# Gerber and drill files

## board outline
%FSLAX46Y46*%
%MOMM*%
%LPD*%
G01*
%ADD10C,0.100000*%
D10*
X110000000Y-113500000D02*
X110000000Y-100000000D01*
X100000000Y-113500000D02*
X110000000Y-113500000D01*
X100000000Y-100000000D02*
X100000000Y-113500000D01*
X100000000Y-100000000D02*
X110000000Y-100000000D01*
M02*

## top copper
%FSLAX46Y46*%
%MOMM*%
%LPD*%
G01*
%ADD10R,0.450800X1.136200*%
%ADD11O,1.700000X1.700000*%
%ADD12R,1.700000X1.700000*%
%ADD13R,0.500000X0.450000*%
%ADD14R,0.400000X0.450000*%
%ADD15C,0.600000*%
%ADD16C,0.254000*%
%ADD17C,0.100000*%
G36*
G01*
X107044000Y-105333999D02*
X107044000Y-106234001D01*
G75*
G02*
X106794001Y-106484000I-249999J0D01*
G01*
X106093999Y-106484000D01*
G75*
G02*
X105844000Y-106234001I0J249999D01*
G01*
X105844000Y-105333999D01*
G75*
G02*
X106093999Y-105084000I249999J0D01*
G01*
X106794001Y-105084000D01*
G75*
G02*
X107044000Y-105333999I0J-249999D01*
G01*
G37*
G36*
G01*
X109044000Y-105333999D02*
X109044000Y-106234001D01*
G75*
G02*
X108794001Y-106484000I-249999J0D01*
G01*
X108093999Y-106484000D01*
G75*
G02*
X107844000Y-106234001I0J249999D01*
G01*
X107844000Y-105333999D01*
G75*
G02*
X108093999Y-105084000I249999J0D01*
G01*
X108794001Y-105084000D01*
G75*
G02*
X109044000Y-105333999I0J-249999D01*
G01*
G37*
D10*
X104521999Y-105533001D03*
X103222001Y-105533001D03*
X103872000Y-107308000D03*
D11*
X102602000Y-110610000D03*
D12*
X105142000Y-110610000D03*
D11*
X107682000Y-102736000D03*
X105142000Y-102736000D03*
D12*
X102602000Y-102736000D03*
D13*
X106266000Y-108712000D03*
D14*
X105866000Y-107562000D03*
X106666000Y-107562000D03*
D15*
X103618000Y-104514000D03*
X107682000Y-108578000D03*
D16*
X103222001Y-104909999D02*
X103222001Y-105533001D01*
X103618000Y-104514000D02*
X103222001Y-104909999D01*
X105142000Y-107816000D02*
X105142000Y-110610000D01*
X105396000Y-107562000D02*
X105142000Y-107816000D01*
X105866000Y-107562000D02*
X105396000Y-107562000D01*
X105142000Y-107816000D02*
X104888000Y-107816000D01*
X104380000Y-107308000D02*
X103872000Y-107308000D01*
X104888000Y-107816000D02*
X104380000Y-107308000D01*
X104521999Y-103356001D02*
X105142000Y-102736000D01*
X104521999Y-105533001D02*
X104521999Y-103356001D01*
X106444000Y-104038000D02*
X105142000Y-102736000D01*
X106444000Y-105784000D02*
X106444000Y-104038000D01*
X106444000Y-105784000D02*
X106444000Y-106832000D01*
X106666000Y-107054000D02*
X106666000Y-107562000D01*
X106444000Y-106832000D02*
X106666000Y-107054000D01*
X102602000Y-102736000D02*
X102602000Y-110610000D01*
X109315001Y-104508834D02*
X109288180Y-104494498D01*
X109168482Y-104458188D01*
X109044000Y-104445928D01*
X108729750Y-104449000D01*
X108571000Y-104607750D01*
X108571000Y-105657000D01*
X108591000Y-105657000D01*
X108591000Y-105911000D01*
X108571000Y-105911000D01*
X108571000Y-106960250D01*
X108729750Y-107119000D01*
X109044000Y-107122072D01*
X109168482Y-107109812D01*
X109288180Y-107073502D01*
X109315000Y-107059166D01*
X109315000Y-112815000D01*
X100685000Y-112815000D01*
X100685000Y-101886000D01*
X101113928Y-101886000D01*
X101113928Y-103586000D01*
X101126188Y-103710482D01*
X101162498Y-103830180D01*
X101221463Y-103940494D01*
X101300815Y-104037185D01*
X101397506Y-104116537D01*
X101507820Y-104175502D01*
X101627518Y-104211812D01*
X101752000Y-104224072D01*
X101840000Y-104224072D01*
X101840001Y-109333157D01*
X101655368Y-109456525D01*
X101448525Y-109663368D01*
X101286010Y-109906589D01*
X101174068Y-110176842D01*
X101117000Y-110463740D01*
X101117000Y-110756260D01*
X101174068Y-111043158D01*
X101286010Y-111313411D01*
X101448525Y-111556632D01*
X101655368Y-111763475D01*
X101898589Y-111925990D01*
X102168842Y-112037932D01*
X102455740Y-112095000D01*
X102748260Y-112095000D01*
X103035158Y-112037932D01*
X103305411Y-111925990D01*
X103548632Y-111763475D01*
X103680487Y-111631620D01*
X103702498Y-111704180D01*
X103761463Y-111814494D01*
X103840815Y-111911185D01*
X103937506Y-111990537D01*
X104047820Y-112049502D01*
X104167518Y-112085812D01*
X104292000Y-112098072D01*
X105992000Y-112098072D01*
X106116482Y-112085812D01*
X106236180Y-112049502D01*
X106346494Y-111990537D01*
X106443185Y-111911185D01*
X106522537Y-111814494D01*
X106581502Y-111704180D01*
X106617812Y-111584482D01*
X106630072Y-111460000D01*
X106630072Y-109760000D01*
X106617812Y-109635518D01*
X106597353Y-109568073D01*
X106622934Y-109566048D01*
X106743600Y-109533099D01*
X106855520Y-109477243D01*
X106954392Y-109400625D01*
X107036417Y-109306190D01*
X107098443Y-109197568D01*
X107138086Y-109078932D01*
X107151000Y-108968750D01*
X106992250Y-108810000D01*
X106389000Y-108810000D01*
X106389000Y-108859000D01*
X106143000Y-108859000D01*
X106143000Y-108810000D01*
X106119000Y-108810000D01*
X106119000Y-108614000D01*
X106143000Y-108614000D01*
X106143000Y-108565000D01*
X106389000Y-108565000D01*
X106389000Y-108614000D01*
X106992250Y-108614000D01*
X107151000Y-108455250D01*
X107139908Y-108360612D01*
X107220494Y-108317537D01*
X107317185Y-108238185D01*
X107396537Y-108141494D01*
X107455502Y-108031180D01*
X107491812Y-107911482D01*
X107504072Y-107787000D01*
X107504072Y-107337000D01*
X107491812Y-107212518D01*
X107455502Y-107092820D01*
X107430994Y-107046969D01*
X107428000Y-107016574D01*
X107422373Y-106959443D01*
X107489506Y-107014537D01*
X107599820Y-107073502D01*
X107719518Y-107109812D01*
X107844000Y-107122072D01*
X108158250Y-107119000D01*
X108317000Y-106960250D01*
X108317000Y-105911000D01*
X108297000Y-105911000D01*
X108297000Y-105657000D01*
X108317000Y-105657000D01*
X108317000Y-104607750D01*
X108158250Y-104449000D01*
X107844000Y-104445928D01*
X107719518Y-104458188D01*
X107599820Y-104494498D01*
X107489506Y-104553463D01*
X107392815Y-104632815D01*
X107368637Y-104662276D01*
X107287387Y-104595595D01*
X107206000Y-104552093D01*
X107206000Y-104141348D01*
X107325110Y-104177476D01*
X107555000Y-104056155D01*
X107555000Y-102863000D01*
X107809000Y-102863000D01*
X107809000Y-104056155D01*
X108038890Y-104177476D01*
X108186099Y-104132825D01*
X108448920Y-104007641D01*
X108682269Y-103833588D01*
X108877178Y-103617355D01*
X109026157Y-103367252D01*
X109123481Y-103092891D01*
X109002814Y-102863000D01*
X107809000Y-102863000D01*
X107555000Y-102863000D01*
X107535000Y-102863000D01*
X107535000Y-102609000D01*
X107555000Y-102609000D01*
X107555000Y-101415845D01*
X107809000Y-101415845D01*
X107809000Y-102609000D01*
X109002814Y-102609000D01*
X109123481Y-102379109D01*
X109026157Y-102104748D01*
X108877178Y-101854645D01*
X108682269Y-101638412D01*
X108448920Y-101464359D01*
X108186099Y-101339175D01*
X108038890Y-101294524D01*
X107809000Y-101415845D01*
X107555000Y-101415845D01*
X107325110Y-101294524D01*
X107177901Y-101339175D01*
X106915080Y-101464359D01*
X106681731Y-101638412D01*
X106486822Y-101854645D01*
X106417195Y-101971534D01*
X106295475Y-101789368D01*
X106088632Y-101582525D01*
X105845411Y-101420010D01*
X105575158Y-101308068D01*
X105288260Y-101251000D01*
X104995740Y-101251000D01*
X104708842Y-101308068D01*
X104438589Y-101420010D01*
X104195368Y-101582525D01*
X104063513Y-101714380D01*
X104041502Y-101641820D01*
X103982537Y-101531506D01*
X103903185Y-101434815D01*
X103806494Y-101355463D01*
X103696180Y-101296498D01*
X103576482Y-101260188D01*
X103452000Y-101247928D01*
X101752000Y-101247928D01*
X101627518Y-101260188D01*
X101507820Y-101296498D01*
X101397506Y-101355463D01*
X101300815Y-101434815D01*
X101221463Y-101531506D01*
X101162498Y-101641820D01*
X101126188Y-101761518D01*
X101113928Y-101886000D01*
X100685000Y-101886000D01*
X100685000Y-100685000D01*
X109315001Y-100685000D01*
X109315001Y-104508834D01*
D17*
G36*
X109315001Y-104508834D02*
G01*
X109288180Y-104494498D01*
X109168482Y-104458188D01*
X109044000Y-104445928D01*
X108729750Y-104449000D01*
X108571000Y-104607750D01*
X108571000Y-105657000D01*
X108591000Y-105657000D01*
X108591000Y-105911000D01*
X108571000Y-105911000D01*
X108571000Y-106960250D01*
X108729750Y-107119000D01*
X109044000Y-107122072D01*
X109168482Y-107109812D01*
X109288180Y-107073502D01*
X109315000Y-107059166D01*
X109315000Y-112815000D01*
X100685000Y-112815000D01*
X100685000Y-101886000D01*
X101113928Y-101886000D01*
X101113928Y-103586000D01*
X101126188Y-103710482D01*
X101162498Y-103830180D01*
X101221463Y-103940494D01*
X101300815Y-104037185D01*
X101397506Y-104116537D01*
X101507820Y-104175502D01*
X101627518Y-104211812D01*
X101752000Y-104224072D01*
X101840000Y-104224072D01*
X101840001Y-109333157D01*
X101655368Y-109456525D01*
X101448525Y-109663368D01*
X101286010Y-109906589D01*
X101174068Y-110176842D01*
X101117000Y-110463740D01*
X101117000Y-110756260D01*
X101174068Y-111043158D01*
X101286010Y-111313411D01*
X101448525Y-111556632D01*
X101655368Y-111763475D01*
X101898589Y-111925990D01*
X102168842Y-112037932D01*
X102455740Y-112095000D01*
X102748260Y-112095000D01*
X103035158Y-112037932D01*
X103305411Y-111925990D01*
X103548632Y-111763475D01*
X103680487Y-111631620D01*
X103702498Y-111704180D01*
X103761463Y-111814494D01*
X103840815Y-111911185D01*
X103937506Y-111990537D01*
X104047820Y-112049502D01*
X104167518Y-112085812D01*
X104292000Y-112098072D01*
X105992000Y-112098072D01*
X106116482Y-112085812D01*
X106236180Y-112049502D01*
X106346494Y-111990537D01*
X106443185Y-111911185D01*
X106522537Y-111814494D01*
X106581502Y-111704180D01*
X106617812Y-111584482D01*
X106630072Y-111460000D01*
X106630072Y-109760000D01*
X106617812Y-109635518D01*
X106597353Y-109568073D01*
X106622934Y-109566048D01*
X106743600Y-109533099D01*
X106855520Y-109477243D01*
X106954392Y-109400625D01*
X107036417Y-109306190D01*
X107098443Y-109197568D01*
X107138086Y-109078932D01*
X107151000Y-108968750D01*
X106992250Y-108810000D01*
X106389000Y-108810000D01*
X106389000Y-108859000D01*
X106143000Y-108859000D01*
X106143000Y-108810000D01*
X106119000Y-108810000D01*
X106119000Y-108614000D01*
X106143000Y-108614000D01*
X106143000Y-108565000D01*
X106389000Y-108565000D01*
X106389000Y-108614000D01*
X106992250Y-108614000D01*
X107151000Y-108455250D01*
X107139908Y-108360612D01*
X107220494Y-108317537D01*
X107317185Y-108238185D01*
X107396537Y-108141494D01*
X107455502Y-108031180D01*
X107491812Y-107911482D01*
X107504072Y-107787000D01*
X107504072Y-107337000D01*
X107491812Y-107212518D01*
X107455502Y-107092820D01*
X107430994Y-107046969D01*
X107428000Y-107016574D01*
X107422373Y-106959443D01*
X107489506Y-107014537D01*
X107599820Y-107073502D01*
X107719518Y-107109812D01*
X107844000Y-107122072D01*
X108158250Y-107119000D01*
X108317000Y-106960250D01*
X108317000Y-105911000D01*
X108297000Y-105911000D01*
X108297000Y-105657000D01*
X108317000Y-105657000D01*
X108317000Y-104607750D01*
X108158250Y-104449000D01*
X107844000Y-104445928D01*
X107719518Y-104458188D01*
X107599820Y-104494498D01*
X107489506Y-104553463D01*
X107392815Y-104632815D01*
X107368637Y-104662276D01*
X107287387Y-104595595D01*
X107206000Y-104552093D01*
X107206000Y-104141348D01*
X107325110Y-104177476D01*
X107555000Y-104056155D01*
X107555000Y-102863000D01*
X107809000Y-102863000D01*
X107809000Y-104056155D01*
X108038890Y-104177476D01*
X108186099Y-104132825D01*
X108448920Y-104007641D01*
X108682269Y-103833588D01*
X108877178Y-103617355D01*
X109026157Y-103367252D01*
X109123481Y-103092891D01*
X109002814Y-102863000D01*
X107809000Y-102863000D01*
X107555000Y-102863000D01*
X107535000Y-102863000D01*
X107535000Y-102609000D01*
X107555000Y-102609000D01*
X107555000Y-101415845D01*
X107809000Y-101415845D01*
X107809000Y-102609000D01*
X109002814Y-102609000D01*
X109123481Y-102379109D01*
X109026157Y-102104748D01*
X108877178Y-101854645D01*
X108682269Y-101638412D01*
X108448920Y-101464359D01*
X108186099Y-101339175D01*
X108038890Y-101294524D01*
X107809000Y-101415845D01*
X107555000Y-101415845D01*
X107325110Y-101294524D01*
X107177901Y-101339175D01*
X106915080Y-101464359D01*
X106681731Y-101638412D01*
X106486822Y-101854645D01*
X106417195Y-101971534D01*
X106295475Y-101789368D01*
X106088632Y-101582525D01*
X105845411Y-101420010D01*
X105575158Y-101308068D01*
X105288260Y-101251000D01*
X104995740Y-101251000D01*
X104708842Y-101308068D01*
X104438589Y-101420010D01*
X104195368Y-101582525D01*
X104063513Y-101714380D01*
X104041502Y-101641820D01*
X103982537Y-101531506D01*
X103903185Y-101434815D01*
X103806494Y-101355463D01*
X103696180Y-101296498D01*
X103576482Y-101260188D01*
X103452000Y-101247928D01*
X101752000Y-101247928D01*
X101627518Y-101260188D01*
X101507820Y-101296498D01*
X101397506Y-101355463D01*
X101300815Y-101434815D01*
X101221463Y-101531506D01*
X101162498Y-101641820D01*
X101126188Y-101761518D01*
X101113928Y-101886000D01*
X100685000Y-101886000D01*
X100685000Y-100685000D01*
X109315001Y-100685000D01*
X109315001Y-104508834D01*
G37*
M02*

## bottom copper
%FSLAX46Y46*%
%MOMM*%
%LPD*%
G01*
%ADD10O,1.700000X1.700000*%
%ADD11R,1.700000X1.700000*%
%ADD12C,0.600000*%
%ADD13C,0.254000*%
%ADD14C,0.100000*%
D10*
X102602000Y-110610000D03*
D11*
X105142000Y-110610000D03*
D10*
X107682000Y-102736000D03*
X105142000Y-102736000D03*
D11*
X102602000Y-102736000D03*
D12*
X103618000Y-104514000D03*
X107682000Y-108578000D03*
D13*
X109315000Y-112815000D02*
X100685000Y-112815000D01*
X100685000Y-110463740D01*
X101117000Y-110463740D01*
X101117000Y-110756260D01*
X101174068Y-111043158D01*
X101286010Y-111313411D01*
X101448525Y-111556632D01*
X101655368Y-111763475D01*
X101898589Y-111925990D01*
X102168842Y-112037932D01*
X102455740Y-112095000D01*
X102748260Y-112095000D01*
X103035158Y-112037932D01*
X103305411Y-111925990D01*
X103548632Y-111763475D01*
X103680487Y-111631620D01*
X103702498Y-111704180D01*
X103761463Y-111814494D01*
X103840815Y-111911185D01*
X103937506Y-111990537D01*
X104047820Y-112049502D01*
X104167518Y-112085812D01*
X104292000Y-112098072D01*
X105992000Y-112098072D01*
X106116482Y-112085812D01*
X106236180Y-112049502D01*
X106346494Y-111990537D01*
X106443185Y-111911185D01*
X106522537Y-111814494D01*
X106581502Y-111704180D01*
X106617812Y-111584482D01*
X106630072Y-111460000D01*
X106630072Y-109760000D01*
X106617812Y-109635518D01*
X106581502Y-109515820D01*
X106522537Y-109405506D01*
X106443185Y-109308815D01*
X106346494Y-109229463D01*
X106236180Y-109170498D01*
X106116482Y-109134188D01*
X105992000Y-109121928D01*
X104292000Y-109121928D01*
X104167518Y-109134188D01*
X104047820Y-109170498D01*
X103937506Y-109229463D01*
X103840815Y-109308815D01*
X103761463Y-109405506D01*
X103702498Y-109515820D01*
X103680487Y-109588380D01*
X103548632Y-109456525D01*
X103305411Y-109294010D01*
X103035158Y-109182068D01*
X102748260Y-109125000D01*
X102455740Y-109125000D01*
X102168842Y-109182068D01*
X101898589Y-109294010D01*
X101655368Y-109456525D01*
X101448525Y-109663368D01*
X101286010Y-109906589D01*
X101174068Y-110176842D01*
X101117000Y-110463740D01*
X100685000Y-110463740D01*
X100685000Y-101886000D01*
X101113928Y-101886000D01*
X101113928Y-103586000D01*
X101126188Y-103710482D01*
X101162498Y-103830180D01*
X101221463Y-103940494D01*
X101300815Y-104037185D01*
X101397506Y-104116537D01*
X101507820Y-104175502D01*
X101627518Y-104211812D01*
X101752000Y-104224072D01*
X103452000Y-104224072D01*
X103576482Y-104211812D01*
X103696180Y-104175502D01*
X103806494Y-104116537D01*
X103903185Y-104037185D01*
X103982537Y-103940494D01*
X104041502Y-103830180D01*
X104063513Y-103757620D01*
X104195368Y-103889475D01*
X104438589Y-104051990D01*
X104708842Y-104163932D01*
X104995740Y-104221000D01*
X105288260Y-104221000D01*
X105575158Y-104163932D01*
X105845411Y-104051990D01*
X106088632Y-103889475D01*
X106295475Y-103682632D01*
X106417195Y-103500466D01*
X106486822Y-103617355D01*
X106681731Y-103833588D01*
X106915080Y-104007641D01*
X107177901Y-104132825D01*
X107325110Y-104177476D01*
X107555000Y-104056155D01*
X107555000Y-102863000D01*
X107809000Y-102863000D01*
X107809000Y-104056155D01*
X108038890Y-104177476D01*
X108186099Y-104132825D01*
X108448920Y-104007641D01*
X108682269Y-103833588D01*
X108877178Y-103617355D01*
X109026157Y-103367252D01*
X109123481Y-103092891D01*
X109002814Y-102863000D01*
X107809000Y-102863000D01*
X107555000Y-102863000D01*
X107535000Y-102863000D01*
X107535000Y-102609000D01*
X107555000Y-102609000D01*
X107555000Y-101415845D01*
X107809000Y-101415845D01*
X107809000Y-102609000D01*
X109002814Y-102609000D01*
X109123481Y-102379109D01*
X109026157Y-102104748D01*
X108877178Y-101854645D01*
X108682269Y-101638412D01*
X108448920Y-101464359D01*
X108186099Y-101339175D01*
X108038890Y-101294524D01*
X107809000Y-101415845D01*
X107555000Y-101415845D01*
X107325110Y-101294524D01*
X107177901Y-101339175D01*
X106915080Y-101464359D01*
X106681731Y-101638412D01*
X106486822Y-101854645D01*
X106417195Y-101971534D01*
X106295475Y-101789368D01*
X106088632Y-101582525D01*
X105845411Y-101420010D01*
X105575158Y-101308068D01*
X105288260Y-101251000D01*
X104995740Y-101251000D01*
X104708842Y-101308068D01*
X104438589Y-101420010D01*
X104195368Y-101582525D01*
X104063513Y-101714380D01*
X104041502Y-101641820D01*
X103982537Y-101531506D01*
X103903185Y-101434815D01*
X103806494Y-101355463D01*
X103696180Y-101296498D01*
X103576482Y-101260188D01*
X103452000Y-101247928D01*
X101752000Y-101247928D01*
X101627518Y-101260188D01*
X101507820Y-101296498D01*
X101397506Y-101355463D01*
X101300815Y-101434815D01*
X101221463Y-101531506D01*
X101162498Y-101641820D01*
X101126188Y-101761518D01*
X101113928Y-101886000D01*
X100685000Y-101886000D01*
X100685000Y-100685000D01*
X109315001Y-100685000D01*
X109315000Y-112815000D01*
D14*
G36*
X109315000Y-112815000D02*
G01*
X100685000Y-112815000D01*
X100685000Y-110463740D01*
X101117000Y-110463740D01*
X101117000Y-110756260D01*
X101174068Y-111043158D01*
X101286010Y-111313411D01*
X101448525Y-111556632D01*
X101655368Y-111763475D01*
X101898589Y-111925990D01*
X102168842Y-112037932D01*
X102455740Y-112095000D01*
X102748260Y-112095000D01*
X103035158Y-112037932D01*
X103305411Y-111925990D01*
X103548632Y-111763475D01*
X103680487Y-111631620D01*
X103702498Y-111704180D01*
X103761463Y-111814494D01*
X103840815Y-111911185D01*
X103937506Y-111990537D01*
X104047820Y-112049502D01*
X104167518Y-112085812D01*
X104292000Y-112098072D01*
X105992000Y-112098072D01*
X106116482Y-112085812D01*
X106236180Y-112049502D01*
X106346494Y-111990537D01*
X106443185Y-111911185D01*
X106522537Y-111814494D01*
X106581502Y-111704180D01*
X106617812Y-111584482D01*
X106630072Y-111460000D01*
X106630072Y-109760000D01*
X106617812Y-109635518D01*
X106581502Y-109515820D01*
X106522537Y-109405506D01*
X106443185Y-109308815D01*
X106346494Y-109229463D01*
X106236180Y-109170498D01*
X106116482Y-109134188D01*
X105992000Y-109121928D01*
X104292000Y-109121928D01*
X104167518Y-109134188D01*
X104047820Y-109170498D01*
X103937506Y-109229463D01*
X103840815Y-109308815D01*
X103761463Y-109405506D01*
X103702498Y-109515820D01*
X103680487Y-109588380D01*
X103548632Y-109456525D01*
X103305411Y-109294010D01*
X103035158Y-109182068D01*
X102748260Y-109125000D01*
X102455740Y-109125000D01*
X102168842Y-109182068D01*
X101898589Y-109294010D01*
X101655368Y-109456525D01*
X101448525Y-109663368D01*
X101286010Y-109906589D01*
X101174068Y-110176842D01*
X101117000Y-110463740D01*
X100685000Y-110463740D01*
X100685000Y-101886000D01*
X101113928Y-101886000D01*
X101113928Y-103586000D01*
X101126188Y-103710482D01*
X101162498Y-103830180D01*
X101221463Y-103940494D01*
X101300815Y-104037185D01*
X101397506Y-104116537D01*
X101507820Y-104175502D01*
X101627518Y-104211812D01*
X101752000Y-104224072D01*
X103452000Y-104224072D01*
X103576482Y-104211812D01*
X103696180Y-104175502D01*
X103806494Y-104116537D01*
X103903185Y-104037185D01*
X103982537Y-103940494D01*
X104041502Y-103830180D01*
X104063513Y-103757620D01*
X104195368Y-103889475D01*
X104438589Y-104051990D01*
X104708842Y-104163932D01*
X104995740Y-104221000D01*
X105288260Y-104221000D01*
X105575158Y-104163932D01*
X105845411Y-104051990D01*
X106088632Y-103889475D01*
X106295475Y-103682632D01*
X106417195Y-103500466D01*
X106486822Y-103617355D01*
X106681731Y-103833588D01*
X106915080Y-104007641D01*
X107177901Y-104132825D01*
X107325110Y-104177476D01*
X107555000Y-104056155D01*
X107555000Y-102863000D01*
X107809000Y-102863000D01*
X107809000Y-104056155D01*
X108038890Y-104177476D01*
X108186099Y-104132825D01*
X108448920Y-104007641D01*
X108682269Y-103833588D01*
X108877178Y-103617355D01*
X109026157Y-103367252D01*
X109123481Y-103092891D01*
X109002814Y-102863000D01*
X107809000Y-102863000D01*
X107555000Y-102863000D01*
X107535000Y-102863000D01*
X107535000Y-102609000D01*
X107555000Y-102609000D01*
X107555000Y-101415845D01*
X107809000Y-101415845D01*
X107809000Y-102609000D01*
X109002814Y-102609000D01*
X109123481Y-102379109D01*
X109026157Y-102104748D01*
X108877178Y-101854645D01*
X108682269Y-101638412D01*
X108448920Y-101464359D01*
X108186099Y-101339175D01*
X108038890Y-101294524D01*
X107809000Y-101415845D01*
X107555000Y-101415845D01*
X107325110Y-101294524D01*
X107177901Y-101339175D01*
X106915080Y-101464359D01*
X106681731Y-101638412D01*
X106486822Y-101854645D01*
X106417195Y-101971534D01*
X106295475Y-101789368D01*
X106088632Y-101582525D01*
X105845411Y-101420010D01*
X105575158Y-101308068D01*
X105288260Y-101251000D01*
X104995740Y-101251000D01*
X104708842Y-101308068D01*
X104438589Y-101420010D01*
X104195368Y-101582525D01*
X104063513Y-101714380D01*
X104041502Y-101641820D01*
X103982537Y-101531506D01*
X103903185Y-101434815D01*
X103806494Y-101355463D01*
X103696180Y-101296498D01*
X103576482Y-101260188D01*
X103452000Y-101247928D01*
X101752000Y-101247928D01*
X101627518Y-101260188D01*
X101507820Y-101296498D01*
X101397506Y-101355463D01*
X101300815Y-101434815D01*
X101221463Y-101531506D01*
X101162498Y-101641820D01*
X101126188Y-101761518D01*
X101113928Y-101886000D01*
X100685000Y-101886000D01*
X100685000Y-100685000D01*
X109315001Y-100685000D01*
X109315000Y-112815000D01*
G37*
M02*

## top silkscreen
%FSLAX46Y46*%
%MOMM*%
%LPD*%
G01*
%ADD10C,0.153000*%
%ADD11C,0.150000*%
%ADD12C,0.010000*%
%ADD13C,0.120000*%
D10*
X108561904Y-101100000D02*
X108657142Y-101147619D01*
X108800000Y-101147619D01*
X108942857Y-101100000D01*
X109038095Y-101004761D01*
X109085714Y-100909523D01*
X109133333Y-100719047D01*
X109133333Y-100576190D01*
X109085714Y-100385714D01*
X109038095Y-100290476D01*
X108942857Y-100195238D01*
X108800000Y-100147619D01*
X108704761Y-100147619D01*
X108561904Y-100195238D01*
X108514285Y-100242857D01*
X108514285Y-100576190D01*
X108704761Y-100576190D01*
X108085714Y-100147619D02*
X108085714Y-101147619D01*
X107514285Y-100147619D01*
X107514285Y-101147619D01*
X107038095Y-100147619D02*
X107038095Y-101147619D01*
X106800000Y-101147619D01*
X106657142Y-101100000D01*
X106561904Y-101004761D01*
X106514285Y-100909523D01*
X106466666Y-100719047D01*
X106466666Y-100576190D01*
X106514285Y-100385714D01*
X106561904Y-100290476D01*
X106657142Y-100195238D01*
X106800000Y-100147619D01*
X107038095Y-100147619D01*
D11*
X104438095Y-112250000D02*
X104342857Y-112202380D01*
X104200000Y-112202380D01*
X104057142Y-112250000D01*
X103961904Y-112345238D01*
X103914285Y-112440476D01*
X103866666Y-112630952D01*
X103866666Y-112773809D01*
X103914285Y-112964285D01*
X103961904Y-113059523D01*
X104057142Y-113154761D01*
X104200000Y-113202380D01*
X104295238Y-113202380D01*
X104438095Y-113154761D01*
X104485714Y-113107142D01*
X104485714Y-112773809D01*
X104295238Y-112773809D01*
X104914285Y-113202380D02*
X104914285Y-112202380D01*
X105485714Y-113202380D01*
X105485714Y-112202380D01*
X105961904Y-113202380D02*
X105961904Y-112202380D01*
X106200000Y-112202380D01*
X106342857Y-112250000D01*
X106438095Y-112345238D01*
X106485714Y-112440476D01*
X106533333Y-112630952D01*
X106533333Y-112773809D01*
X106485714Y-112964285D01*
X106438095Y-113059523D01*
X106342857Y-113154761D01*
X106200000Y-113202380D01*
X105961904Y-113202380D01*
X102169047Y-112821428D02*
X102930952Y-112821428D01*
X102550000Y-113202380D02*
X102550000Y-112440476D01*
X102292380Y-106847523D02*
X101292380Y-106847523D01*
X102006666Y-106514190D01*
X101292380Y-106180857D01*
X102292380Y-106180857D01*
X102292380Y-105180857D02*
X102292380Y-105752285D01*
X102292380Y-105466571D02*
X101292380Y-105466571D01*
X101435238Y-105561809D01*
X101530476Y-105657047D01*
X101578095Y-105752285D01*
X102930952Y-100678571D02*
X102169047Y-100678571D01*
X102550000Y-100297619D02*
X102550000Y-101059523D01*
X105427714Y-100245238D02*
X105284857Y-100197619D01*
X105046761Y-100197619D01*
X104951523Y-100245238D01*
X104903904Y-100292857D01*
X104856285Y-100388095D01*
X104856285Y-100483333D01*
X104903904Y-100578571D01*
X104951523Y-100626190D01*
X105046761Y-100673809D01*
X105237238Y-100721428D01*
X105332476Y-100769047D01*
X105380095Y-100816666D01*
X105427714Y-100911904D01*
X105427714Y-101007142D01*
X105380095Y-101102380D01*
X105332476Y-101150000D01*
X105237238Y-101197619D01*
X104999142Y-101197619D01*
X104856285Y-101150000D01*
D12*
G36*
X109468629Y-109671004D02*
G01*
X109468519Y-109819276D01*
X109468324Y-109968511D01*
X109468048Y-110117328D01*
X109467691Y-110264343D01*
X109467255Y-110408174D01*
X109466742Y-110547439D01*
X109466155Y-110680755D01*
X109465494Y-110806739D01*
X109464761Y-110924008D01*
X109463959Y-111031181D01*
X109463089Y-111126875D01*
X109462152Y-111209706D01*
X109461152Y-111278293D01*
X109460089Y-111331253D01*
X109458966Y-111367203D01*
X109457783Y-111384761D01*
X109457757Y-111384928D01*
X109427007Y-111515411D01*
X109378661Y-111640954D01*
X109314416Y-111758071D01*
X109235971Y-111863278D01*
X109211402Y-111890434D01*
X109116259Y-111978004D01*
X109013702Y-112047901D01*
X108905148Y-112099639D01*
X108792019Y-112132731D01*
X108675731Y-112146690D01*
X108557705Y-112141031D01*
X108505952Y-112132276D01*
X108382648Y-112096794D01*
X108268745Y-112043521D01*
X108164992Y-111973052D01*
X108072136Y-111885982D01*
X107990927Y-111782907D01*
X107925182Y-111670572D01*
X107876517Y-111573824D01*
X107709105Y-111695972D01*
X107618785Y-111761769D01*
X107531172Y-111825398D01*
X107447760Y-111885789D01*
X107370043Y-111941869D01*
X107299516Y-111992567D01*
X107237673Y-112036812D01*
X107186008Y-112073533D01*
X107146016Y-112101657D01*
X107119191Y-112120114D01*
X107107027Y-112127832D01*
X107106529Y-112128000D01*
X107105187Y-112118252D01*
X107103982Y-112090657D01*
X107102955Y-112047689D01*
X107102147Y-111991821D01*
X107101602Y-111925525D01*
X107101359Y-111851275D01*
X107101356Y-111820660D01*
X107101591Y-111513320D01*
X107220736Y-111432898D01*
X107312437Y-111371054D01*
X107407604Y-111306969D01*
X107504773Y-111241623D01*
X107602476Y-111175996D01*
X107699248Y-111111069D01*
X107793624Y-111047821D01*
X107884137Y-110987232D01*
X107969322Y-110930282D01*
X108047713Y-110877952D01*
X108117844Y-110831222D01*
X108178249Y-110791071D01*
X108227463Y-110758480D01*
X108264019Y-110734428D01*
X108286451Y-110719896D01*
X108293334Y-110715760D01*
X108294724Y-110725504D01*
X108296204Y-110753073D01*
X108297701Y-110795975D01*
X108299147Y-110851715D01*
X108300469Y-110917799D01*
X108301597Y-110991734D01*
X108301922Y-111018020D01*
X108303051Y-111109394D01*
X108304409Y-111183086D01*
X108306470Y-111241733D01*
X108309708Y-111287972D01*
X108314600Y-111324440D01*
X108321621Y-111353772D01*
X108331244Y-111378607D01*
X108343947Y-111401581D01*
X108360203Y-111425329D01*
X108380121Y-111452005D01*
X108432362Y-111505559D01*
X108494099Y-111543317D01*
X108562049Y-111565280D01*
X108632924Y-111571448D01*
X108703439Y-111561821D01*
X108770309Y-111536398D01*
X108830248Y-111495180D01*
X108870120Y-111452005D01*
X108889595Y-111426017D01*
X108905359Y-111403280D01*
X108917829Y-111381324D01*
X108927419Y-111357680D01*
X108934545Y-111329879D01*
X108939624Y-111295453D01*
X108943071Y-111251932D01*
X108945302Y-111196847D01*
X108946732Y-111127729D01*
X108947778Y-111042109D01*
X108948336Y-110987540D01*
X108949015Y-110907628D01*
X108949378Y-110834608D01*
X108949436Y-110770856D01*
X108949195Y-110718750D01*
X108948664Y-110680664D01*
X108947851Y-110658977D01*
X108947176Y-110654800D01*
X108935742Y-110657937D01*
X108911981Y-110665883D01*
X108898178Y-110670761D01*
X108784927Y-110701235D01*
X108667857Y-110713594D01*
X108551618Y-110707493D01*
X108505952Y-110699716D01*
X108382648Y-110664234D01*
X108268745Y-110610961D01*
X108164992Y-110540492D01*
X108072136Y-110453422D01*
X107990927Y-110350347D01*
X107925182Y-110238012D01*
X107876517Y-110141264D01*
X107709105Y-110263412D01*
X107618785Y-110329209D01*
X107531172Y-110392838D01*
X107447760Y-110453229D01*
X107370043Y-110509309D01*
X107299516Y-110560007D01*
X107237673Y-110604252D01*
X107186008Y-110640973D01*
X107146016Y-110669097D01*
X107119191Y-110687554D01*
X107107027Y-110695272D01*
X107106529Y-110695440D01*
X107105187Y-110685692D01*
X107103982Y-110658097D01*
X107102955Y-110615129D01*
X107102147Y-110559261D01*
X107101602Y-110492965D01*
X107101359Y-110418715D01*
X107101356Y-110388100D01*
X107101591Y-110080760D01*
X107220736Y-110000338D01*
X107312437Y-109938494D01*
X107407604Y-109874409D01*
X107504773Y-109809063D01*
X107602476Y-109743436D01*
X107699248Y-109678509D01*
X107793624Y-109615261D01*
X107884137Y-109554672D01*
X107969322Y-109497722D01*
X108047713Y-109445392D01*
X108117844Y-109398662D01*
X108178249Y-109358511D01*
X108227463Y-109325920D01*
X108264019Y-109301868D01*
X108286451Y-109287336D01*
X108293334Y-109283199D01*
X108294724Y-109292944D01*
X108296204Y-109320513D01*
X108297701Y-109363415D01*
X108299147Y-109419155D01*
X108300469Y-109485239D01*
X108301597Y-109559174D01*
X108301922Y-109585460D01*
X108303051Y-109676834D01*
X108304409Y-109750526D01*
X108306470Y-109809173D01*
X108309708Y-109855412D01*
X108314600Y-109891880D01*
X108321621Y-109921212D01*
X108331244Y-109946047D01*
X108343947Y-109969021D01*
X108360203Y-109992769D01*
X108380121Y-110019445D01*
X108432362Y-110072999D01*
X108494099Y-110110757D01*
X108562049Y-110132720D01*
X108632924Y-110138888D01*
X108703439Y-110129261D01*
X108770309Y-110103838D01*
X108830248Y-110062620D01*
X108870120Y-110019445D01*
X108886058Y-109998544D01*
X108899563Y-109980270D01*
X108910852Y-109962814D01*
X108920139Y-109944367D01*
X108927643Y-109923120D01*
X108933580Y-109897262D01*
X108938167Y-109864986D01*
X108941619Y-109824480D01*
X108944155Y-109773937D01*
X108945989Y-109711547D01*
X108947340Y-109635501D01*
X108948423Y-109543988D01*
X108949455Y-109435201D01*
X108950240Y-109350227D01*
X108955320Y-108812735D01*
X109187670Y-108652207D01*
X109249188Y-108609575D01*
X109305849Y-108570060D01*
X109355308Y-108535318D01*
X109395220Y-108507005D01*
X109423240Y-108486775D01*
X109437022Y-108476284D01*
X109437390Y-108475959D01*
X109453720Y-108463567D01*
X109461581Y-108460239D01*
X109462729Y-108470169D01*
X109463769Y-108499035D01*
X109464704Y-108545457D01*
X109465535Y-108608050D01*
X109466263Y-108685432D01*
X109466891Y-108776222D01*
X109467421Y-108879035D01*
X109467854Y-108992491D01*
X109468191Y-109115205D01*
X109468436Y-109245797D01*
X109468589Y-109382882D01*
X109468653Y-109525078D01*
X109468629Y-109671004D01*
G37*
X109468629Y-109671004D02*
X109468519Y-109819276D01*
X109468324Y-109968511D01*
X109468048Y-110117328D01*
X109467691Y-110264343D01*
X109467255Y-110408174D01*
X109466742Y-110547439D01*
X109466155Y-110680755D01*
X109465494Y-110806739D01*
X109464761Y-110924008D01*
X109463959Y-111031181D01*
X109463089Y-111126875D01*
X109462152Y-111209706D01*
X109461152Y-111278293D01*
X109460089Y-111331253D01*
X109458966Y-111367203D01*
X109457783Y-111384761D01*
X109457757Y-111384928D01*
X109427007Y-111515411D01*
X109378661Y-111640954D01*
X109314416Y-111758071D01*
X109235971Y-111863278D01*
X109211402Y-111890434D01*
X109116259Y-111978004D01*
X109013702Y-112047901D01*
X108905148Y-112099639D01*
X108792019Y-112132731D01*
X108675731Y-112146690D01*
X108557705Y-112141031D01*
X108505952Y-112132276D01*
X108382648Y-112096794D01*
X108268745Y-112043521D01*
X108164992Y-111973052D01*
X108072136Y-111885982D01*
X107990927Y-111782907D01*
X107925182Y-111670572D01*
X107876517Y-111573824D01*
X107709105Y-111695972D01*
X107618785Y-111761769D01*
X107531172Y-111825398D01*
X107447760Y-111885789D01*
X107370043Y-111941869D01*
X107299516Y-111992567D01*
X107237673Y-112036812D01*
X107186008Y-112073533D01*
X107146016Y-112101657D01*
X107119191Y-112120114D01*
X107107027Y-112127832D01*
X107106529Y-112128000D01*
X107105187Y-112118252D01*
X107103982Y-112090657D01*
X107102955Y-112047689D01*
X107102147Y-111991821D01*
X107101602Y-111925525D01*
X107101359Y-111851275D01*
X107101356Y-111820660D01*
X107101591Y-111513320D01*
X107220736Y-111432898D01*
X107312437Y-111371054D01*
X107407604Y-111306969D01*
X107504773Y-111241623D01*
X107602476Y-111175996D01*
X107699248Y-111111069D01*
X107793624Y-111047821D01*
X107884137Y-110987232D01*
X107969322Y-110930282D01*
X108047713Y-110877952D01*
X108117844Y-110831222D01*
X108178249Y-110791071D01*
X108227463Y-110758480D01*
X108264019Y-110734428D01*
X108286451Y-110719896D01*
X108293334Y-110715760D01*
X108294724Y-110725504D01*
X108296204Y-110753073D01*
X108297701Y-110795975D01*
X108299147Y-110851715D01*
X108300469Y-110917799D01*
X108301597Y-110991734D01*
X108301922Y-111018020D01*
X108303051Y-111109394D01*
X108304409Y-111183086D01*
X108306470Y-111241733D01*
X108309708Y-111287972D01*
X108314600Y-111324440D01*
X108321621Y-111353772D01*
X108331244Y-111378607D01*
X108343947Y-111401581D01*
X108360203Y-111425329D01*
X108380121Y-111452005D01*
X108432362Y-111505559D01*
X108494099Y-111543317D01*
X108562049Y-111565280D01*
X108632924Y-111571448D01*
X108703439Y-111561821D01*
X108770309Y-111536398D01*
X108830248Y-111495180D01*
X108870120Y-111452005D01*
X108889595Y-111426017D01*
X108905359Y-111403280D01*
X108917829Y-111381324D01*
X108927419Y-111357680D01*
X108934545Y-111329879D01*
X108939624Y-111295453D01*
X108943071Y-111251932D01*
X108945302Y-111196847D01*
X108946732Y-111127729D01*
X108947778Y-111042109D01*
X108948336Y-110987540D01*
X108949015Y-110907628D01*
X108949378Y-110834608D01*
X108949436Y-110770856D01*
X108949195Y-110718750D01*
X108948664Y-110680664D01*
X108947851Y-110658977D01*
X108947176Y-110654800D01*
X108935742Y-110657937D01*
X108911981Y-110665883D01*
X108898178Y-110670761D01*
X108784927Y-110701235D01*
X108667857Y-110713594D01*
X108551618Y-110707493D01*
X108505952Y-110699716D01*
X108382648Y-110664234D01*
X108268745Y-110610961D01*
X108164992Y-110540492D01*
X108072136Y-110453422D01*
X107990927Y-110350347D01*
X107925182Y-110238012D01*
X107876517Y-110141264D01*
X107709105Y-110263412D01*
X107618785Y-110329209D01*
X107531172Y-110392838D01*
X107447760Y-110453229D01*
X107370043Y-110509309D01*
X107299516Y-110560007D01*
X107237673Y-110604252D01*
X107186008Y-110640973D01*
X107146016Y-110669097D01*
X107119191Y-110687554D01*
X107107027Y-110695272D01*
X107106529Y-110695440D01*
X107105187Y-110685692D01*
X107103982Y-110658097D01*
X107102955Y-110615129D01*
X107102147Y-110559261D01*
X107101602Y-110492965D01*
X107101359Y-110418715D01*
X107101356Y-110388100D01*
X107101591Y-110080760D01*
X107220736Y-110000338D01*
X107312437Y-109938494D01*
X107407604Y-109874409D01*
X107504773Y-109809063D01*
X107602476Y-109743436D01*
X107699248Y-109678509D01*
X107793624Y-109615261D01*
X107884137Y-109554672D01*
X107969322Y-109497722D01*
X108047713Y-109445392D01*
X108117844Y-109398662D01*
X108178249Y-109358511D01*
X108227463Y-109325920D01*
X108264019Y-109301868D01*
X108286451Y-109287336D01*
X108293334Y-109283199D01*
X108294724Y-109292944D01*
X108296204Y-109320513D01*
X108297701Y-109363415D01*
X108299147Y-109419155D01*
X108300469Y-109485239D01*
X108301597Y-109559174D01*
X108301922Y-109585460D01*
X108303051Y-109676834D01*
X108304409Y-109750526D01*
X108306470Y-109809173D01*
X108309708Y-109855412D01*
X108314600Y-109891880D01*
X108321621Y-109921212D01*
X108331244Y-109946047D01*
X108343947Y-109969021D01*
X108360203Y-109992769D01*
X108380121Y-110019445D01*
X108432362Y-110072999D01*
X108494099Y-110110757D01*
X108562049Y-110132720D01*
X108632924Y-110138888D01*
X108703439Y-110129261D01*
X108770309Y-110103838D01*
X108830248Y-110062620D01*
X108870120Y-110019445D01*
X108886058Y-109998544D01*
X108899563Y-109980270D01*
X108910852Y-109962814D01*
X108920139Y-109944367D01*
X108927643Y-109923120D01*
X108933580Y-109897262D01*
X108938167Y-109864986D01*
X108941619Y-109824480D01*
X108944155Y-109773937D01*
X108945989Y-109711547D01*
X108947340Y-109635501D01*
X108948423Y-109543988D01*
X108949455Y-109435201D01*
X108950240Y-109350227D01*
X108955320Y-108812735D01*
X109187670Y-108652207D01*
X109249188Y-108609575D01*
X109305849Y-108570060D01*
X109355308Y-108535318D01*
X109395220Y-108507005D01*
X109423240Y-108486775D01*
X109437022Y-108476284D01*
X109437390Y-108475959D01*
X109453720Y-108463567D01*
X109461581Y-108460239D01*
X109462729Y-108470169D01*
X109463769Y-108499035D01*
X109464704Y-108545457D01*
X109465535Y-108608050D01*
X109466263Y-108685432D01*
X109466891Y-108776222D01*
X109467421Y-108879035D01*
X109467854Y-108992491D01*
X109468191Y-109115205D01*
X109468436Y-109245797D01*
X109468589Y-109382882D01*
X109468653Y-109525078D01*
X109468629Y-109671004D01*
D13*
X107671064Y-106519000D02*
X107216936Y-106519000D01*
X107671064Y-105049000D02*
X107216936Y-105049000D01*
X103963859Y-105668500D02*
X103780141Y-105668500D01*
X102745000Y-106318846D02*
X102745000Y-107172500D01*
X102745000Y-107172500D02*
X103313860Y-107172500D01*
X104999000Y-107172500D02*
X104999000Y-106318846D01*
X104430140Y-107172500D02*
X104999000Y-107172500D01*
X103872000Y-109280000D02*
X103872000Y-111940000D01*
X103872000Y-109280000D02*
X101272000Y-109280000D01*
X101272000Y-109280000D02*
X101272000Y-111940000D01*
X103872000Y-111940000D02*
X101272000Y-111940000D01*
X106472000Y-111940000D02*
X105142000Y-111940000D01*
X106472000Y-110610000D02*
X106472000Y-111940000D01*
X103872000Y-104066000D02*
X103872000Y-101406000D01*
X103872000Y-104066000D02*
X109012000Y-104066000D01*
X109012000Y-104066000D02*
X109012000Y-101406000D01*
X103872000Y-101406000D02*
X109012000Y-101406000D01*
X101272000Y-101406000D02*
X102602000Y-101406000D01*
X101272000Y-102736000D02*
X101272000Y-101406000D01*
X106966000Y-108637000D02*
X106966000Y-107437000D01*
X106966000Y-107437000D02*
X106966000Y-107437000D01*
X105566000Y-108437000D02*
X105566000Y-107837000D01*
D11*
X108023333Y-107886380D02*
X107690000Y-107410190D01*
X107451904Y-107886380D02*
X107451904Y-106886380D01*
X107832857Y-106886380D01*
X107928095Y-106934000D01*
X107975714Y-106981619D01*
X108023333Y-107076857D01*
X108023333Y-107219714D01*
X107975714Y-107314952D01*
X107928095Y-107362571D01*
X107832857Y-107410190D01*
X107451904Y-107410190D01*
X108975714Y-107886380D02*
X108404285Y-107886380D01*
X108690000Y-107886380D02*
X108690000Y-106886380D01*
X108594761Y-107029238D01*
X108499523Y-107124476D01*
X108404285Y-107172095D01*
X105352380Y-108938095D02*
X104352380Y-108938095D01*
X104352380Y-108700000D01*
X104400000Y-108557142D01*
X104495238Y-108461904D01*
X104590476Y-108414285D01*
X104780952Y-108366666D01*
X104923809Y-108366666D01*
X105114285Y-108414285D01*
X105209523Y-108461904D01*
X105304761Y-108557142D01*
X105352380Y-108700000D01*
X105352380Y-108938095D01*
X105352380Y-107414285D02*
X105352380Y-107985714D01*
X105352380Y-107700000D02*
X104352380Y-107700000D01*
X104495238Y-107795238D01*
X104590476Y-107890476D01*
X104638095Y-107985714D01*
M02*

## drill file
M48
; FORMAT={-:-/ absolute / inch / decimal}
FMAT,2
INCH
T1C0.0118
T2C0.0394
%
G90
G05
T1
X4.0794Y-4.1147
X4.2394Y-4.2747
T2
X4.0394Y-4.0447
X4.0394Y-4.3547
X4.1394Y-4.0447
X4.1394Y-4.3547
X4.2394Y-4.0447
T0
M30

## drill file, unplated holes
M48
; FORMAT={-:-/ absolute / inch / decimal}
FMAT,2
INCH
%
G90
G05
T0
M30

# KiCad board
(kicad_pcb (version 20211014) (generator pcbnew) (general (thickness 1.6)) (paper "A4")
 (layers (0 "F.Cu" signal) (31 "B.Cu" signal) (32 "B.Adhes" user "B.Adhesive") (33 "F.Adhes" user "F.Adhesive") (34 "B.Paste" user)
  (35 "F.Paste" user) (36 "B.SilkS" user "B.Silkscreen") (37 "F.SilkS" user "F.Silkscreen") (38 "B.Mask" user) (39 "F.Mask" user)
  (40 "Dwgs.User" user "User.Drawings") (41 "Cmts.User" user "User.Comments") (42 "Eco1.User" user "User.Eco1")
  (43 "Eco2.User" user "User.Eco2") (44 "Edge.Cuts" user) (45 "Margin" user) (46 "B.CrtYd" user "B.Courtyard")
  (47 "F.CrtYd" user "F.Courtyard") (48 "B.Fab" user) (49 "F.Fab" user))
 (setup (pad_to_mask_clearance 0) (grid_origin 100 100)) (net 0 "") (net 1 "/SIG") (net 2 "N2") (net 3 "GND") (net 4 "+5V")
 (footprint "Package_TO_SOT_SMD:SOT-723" (layer "F.Cu") (at 106.266 108.137 -90)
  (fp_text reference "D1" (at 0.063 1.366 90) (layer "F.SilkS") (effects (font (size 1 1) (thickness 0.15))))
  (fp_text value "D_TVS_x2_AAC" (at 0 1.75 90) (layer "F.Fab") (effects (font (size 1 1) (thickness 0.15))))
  (fp_line (start 0.5 -0.7) (end -0.7 -0.7) (layer "F.SilkS") (width 0.12))
  (fp_line (start -0.7 -0.7) (end -0.7 -0.7) (layer "F.SilkS") (width 0.12))
  (fp_line (start 0.3 0.7) (end -0.3 0.7) (layer "F.SilkS") (width 0.12))
  (pad "1" smd rect locked (at -0.575 -0.4 270) (size 0.45 0.4) (layers "F.Cu" "F.Paste" "F.Mask") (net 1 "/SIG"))
  (pad "2" smd rect locked (at -0.575 0.4 270) (size 0.45 0.4) (layers "F.Cu" "F.Paste" "F.Mask") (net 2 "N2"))
  (pad "3" smd rect locked (at 0.575 0 270) (size 0.45 0.5) (layers "F.Cu" "F.Paste" "F.Mask") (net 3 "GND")))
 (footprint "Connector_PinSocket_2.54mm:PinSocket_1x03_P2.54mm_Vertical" (layer "F.Cu") (at 102.602 102.736 90)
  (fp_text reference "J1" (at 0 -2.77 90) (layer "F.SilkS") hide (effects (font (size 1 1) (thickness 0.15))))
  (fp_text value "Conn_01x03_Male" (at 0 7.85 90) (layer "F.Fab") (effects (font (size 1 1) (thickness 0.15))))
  (fp_line (start 1.33 -1.33) (end 1.33 0) (layer "F.SilkS") (width 0.12))
  (fp_line (start -1.33 1.27) (end 1.33 1.27) (layer "F.SilkS") (width 0.12))
  (fp_line (start -1.33 1.27) (end -1.33 6.41) (layer "F.SilkS") (width 0.12))
  (fp_line (start 1.33 1.27) (end 1.33 6.41) (layer "F.SilkS") (width 0.12))
  (fp_line (start 0 -1.33) (end 1.33 -1.33) (layer "F.SilkS") (width 0.12))
  (fp_line (start -1.33 6.41) (end 1.33 6.41) (layer "F.SilkS") (width 0.12))
  (pad "1" thru_hole rect locked (at 0 0 90) (size 1.7 1.7) (drill 1) (layers *.Cu *.Mask) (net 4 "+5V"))
  (pad "2" thru_hole oval locked (at 0 2.54 90) (size 1.7 1.7) (drill 1) (layers *.Cu *.Mask) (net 1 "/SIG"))
  (pad "3" thru_hole oval locked (at 0 5.08 90) (size 1.7 1.7) (drill 1) (layers *.Cu *.Mask) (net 3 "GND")))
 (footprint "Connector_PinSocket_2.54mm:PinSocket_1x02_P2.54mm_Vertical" (layer "F.Cu") (at 105.142 110.61 -90)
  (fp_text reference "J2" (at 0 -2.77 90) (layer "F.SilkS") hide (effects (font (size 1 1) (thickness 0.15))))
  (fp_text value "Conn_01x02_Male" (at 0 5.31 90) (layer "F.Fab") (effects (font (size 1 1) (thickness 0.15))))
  (fp_line (start 1.33 1.27) (end 1.33 3.87) (layer "F.SilkS") (width 0.12))
  (fp_line (start -1.33 1.27) (end -1.33 3.87) (layer "F.SilkS") (width 0.12))
  (fp_line (start -1.33 1.27) (end 1.33 1.27) (layer "F.SilkS") (width 0.12))
  (fp_line (start 1.33 -1.33) (end 1.33 0) (layer "F.SilkS") (width 0.12))
  (fp_line (start -1.33 3.87) (end 1.33 3.87) (layer "F.SilkS") (width 0.12))
  (fp_line (start 0 -1.33) (end 1.33 -1.33) (layer "F.SilkS") (width 0.12))
  (pad "1" thru_hole rect locked (at 0 0 270) (size 1.7 1.7) (drill 1) (layers *.Cu *.Mask) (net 2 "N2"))
  (pad "2" thru_hole oval locked (at 0 2.54 270) (size 1.7 1.7) (drill 1) (layers *.Cu *.Mask) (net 4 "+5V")))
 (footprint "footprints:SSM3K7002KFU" (layer "F.Cu") (at 103.872 106.4205 180)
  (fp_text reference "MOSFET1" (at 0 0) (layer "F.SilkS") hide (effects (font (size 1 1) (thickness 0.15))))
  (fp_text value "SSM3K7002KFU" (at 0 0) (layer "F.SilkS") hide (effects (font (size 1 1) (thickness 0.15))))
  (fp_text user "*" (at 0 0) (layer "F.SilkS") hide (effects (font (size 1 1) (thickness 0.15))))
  (fp_line (start -1.127 -0.752) (end -1.127 0.101654) (layer "F.SilkS") (width 0.12))
  (fp_line (start -0.55814 -0.752) (end -1.127 -0.752) (layer "F.SilkS") (width 0.12))
  (fp_line (start 1.127 0.101654) (end 1.127 -0.752) (layer "F.SilkS") (width 0.12))
  (fp_line (start 1.127 -0.752) (end 0.55814 -0.752) (layer "F.SilkS") (width 0.12))
  (fp_line (start -0.091859 0.752) (end 0.091859 0.752) (layer "F.SilkS") (width 0.12))
  (pad "1" smd rect locked (at -0.649999 0.887499 180) (size 0.4508 1.1362) (layers "F.Cu" "F.Paste" "F.Mask") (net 1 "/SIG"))
  (pad "2" smd rect locked (at 0.649999 0.887499 180) (size 0.4508 1.1362) (layers "F.Cu" "F.Paste" "F.Mask") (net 3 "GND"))
  (pad "3" smd rect locked (at 0 -0.8875 180) (size 0.4508 1.1362) (layers "F.Cu" "F.Paste" "F.Mask") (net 2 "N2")))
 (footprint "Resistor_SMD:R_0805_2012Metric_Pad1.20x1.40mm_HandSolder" (layer "F.Cu") (at 107.444 105.784 180)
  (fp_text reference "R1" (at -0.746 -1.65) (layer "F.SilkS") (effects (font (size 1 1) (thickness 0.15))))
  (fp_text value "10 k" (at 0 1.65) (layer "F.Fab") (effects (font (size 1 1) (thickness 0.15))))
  (fp_line (start -0.227064 -0.735) (end 0.227064 -0.735) (layer "F.SilkS") (width 0.12))
  (fp_line (start -0.227064 0.735) (end 0.227064 0.735) (layer "F.SilkS") (width 0.12))
  (pad "1" smd roundrect locked (at -1 0 180) (size 1.2 1.4) (layers "F.Cu" "F.Paste" "F.Mask") (roundrect_rratio 0.2083325) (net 3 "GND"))
  (pad "2" smd roundrect locked (at 1 0 180) (size 1.2 1.4) (layers "F.Cu" "F.Paste" "F.Mask") (roundrect_rratio 0.2083325) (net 1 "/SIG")))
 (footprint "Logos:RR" (layer "F.Cu") (at 115.1 108.25)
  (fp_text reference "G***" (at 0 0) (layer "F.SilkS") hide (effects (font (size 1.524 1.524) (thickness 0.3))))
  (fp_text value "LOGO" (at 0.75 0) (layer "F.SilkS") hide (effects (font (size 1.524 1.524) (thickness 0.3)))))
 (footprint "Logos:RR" (layer "F.Cu") (at 116.4 110.45)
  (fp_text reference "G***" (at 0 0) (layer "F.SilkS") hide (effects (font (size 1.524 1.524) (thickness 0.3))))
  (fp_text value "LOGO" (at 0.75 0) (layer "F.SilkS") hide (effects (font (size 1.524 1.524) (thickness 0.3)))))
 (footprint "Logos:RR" (layer "F.Cu") (at 108.3 110.35 -90)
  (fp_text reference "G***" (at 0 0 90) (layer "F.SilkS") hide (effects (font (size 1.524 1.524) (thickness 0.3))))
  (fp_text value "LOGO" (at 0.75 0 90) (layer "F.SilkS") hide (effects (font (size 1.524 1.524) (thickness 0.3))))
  (fp_poly
   (pts (xy -0.678996 -1.168629) (xy -0.530724 -1.168519) (xy -0.381489 -1.168324) (xy -0.232672 -1.168048) (xy -0.085657 -1.167691)
    (xy 0.058174 -1.167255) (xy 0.197439 -1.166742) (xy 0.330755 -1.166155) (xy 0.456739 -1.165494) (xy 0.574008 -1.164761)
    (xy 0.681181 -1.163959) (xy 0.776875 -1.163089) (xy 0.859706 -1.162152) (xy 0.928293 -1.161152) (xy 0.981253 -1.160089)
    (xy 1.017203 -1.158966) (xy 1.034761 -1.157783) (xy 1.034928 -1.157757) (xy 1.165411 -1.127007) (xy 1.290954 -1.078661)
    (xy 1.408071 -1.014416) (xy 1.513278 -0.935971) (xy 1.540434 -0.911402) (xy 1.628004 -0.816259) (xy 1.697901 -0.713702)
    (xy 1.749639 -0.605148) (xy 1.782731 -0.492019) (xy 1.79669 -0.375731) (xy 1.791031 -0.257705) (xy 1.782276 -0.205952)
    (xy 1.746794 -0.082648) (xy 1.693521 0.031255) (xy 1.623052 0.135008) (xy 1.535982 0.227864) (xy 1.432907 0.309073)
    (xy 1.320572 0.374818) (xy 1.223824 0.423483) (xy 1.345972 0.590895) (xy 1.411769 0.681215) (xy 1.475398 0.768828) (xy 1.535789 0.85224)
    (xy 1.591869 0.929957) (xy 1.642567 1.000484) (xy 1.686812 1.062327) (xy 1.723533 1.113992) (xy 1.751657 1.153984)
    (xy 1.770114 1.180809) (xy 1.777832 1.192973) (xy 1.778 1.193471) (xy 1.768252 1.194813) (xy 1.740657 1.196018) (xy 1.697689 1.197045)
    (xy 1.641821 1.197853) (xy 1.575525 1.198398) (xy 1.501275 1.198641) (xy 1.47066 1.198644) (xy 1.16332 1.198409) (xy 1.082898 1.079264)
    (xy 1.021054 0.987563) (xy 0.956969 0.892396) (xy 0.891623 0.795227) (xy 0.825996 0.697524) (xy 0.761069 0.600752)
    (xy 0.697821 0.506376) (xy 0.637232 0.415863) (xy 0.580282 0.330678) (xy 0.527952 0.252287) (xy 0.481222 0.182156)
    (xy 0.441071 0.121751) (xy 0.40848 0.072537) (xy 0.384428 0.035981) (xy 0.369896 0.013549) (xy 0.36576 0.006666) (xy 0.375504 0.005276)
    (xy 0.403073 0.003796) (xy 0.445975 0.002299) (xy 0.501715 0.000853) (xy 0.567799 -0.000469) (xy 0.641734 -0.001597)
    (xy 0.66802 -0.001922) (xy 0.759394 -0.003051) (xy 0.833086 -0.004409) (xy 0.891733 -0.00647) (xy 0.937972 -0.009708)
    (xy 0.97444 -0.0146) (xy 1.003772 -0.021621) (xy 1.028607 -0.031244) (xy 1.051581 -0.043947) (xy 1.075329 -0.060203)
    (xy 1.102005 -0.080121) (xy 1.155559 -0.132362) (xy 1.193317 -0.194099) (xy 1.21528 -0.262049) (xy 1.221448 -0.332924)
    (xy 1.211821 -0.403439) (xy 1.186398 -0.470309) (xy 1.14518 -0.530248) (xy 1.102005 -0.57012) (xy 1.076017 -0.589595)
    (xy 1.05328 -0.605359) (xy 1.031324 -0.617829) (xy 1.00768 -0.627419) (xy 0.979879 -0.634545) (xy 0.945453 -0.639624)
    (xy 0.901932 -0.643071) (xy 0.846847 -0.645302) (xy 0.777729 -0.646732) (xy 0.692109 -0.647778) (xy 0.63754 -0.648336)
    (xy 0.557628 -0.649015) (xy 0.484608 -0.649378) (xy 0.420856 -0.649436) (xy 0.36875 -0.649195) (xy 0.330664 -0.648664)
    (xy 0.308977 -0.647851) (xy 0.3048 -0.647176) (xy 0.307937 -0.635742) (xy 0.315883 -0.611981) (xy 0.320761 -0.598178)
    (xy 0.351235 -0.484927) (xy 0.363594 -0.367857) (xy 0.357493 -0.251618) (xy 0.349716 -0.205952) (xy 0.314234 -0.082648)
    (xy 0.260961 0.031255) (xy 0.190492 0.135008) (xy 0.103422 0.227864) (xy 0.000347 0.309073) (xy -0.111988 0.374818)
    (xy -0.208736 0.423483) (xy -0.086588 0.590895) (xy -0.020791 0.681215) (xy 0.042838 0.768828) (xy 0.103229 0.85224)
    (xy 0.159309 0.929957) (xy 0.210007 1.000484) (xy 0.254252 1.062327) (xy 0.290973 1.113992) (xy 0.319097 1.153984)
    (xy 0.337554 1.180809) (xy 0.345272 1.192973) (xy 0.34544 1.193471) (xy 0.335692 1.194813) (xy 0.308097 1.196018) (xy 0.265129 1.197045)
    (xy 0.209261 1.197853) (xy 0.142965 1.198398) (xy 0.068715 1.198641) (xy 0.0381 1.198644) (xy -0.26924 1.198409) (xy -0.349662 1.079264)
    (xy -0.411506 0.987563) (xy -0.475591 0.892396) (xy -0.540937 0.795227) (xy -0.606564 0.697524) (xy -0.671491 0.600752)
    (xy -0.734739 0.506376) (xy -0.795328 0.415863) (xy -0.852278 0.330678) (xy -0.904608 0.252287) (xy -0.951338 0.182156)
    (xy -0.991489 0.121751) (xy -1.02408 0.072537) (xy -1.048132 0.035981) (xy -1.062664 0.013549) (xy -1.066801 0.006666)
    (xy -1.057056 0.005276) (xy -1.029487 0.003796) (xy -0.986585 0.002299) (xy -0.930845 0.000853) (xy -0.864761 -0.000469)
    (xy -0.790826 -0.001597) (xy -0.76454 -0.001922) (xy -0.673166 -0.003051) (xy -0.599474 -0.004409) (xy -0.540827 -0.00647)
    (xy -0.494588 -0.009708) (xy -0.45812 -0.0146) (xy -0.428788 -0.021621) (xy -0.403953 -0.031244) (xy -0.380979 -0.043947)
    (xy -0.357231 -0.060203) (xy -0.330555 -0.080121) (xy -0.277001 -0.132362) (xy -0.239243 -0.194099) (xy -0.21728 -0.262049)
    (xy -0.211112 -0.332924) (xy -0.220739 -0.403439) (xy -0.246162 -0.470309) (xy -0.28738 -0.530248) (xy -0.330555 -0.57012)
    (xy -0.351456 -0.586058) (xy -0.36973 -0.599563) (xy -0.387186 -0.610852) (xy -0.405633 -0.620139) (xy -0.42688 -0.627643)
    (xy -0.452738 -0.63358) (xy -0.485014 -0.638167) (xy -0.52552 -0.641619) (xy -0.576063 -0.644155) (xy -0.638453 -0.645989)
    (xy -0.714499 -0.64734) (xy -0.806012 -0.648423) (xy -0.914799 -0.649455) (xy -0.999773 -0.65024) (xy -1.537265 -0.65532)
    (xy -1.697793 -0.88767) (xy -1.740425 -0.949188) (xy -1.77994 -1.005849) (xy -1.814682 -1.055308) (xy -1.842995 -1.09522)
    (xy -1.863225 -1.12324) (xy -1.873716 -1.137022) (xy -1.874041 -1.13739) (xy -1.886433 -1.15372) (xy -1.889761 -1.161581)
    (xy -1.879831 -1.162729) (xy -1.850965 -1.163769) (xy -1.804543 -1.164704) (xy -1.74195 -1.165535) (xy -1.664568 -1.166263)
    (xy -1.573778 -1.166891) (xy -1.470965 -1.167421) (xy -1.357509 -1.167854) (xy -1.234795 -1.168191) (xy -1.104203 -1.168436)
    (xy -0.967118 -1.168589) (xy -0.824922 -1.168653) (xy -0.678996 -1.168629))
   (layer "F.SilkS") (width 0.01) (fill solid)))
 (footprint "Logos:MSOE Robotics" (layer "B.Cu") (at 104.5 106.45 -90)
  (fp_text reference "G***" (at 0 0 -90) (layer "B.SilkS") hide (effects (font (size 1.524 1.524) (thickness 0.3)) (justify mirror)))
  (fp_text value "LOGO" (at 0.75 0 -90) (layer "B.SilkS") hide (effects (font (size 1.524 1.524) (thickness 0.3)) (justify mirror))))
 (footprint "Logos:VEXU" (layer "B.Cu") (at 107.85 105.65 -90)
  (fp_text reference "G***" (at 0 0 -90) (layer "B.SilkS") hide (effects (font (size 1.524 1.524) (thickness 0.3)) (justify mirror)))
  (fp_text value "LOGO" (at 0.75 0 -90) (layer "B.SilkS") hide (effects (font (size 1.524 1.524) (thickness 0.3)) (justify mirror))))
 (gr_line (start 100 113.5) (end 110 113.5) (layer "Edge.Cuts") (width 0.1))
 (gr_line (start 110 113.5) (end 110 100) (layer "Edge.Cuts") (width 0.1))
 (gr_line (start 100 100) (end 110 100) (layer "Edge.Cuts") (width 0.1))
 (gr_line (start 100 100) (end 100 113.5) (layer "Edge.Cuts") (width 0.1))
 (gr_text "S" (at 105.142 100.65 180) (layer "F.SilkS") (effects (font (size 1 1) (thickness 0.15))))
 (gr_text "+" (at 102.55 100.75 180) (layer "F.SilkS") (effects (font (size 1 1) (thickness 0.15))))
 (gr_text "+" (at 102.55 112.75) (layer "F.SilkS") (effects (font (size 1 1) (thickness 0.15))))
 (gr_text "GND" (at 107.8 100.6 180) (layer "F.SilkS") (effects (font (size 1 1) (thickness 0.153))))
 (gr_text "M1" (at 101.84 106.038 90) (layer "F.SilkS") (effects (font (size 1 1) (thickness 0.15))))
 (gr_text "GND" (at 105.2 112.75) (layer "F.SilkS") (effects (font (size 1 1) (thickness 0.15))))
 (segment (start 103.222001 104.909999) (end 103.222001 105.533001) (width 0.254) (layer "F.Cu") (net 3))
 (segment (start 103.618 104.514) (end 103.222001 104.909999) (width 0.254) (layer "F.Cu") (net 3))
 (via (at 107.682 108.578) (size 0.6) (drill 0.3) (layers "F.Cu" "B.Cu") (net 3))
 (via (at 103.618 104.514) (size 0.6) (drill 0.3) (layers "F.Cu" "B.Cu") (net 3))
 (segment (start 104.888 107.816) (end 104.38 107.308) (width 0.254) (layer "F.Cu") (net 2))
 (segment (start 105.396 107.562) (end 105.142 107.816) (width 0.254) (layer "F.Cu") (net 2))
 (segment (start 105.866 107.562) (end 105.396 107.562) (width 0.254) (layer "F.Cu") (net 2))
 (segment (start 104.38 107.308) (end 103.872 107.308) (width 0.254) (layer "F.Cu") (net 2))
 (segment (start 105.142 107.816) (end 104.888 107.816) (width 0.254) (layer "F.Cu") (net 2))
 (segment (start 105.142 107.816) (end 105.142 110.61) (width 0.254) (layer "F.Cu") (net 2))
 (segment (start 106.444 106.832) (end 106.666 107.054) (width 0.254) (layer "F.Cu") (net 1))
 (segment (start 106.666 107.054) (end 106.666 107.562) (width 0.254) (layer "F.Cu") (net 1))
 (segment (start 104.521999 105.533001) (end 104.521999 103.356001) (width 0.254) (layer "F.Cu") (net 1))
 (segment (start 104.521999 103.356001) (end 105.142 102.736) (width 0.254) (layer "F.Cu") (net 1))
 (segment (start 106.444 105.784) (end 106.444 106.832) (width 0.254) (layer "F.Cu") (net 1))
 (segment (start 106.444 104.038) (end 105.142 102.736) (width 0.254) (layer "F.Cu") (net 1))
 (segment (start 106.444 105.784) (end 106.444 104.038) (width 0.254) (layer "F.Cu") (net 1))
 (segment (start 102.602 102.736) (end 102.602 110.61) (width 0.254) (layer "F.Cu") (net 4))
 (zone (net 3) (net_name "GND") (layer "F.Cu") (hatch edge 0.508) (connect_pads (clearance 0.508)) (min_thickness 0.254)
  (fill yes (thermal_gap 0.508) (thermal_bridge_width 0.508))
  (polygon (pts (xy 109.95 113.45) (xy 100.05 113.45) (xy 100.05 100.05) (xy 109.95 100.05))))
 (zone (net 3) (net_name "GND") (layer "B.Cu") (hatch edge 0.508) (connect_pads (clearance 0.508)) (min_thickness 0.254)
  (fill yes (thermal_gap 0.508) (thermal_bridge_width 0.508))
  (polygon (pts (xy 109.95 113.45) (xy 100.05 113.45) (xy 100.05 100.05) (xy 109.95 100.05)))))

